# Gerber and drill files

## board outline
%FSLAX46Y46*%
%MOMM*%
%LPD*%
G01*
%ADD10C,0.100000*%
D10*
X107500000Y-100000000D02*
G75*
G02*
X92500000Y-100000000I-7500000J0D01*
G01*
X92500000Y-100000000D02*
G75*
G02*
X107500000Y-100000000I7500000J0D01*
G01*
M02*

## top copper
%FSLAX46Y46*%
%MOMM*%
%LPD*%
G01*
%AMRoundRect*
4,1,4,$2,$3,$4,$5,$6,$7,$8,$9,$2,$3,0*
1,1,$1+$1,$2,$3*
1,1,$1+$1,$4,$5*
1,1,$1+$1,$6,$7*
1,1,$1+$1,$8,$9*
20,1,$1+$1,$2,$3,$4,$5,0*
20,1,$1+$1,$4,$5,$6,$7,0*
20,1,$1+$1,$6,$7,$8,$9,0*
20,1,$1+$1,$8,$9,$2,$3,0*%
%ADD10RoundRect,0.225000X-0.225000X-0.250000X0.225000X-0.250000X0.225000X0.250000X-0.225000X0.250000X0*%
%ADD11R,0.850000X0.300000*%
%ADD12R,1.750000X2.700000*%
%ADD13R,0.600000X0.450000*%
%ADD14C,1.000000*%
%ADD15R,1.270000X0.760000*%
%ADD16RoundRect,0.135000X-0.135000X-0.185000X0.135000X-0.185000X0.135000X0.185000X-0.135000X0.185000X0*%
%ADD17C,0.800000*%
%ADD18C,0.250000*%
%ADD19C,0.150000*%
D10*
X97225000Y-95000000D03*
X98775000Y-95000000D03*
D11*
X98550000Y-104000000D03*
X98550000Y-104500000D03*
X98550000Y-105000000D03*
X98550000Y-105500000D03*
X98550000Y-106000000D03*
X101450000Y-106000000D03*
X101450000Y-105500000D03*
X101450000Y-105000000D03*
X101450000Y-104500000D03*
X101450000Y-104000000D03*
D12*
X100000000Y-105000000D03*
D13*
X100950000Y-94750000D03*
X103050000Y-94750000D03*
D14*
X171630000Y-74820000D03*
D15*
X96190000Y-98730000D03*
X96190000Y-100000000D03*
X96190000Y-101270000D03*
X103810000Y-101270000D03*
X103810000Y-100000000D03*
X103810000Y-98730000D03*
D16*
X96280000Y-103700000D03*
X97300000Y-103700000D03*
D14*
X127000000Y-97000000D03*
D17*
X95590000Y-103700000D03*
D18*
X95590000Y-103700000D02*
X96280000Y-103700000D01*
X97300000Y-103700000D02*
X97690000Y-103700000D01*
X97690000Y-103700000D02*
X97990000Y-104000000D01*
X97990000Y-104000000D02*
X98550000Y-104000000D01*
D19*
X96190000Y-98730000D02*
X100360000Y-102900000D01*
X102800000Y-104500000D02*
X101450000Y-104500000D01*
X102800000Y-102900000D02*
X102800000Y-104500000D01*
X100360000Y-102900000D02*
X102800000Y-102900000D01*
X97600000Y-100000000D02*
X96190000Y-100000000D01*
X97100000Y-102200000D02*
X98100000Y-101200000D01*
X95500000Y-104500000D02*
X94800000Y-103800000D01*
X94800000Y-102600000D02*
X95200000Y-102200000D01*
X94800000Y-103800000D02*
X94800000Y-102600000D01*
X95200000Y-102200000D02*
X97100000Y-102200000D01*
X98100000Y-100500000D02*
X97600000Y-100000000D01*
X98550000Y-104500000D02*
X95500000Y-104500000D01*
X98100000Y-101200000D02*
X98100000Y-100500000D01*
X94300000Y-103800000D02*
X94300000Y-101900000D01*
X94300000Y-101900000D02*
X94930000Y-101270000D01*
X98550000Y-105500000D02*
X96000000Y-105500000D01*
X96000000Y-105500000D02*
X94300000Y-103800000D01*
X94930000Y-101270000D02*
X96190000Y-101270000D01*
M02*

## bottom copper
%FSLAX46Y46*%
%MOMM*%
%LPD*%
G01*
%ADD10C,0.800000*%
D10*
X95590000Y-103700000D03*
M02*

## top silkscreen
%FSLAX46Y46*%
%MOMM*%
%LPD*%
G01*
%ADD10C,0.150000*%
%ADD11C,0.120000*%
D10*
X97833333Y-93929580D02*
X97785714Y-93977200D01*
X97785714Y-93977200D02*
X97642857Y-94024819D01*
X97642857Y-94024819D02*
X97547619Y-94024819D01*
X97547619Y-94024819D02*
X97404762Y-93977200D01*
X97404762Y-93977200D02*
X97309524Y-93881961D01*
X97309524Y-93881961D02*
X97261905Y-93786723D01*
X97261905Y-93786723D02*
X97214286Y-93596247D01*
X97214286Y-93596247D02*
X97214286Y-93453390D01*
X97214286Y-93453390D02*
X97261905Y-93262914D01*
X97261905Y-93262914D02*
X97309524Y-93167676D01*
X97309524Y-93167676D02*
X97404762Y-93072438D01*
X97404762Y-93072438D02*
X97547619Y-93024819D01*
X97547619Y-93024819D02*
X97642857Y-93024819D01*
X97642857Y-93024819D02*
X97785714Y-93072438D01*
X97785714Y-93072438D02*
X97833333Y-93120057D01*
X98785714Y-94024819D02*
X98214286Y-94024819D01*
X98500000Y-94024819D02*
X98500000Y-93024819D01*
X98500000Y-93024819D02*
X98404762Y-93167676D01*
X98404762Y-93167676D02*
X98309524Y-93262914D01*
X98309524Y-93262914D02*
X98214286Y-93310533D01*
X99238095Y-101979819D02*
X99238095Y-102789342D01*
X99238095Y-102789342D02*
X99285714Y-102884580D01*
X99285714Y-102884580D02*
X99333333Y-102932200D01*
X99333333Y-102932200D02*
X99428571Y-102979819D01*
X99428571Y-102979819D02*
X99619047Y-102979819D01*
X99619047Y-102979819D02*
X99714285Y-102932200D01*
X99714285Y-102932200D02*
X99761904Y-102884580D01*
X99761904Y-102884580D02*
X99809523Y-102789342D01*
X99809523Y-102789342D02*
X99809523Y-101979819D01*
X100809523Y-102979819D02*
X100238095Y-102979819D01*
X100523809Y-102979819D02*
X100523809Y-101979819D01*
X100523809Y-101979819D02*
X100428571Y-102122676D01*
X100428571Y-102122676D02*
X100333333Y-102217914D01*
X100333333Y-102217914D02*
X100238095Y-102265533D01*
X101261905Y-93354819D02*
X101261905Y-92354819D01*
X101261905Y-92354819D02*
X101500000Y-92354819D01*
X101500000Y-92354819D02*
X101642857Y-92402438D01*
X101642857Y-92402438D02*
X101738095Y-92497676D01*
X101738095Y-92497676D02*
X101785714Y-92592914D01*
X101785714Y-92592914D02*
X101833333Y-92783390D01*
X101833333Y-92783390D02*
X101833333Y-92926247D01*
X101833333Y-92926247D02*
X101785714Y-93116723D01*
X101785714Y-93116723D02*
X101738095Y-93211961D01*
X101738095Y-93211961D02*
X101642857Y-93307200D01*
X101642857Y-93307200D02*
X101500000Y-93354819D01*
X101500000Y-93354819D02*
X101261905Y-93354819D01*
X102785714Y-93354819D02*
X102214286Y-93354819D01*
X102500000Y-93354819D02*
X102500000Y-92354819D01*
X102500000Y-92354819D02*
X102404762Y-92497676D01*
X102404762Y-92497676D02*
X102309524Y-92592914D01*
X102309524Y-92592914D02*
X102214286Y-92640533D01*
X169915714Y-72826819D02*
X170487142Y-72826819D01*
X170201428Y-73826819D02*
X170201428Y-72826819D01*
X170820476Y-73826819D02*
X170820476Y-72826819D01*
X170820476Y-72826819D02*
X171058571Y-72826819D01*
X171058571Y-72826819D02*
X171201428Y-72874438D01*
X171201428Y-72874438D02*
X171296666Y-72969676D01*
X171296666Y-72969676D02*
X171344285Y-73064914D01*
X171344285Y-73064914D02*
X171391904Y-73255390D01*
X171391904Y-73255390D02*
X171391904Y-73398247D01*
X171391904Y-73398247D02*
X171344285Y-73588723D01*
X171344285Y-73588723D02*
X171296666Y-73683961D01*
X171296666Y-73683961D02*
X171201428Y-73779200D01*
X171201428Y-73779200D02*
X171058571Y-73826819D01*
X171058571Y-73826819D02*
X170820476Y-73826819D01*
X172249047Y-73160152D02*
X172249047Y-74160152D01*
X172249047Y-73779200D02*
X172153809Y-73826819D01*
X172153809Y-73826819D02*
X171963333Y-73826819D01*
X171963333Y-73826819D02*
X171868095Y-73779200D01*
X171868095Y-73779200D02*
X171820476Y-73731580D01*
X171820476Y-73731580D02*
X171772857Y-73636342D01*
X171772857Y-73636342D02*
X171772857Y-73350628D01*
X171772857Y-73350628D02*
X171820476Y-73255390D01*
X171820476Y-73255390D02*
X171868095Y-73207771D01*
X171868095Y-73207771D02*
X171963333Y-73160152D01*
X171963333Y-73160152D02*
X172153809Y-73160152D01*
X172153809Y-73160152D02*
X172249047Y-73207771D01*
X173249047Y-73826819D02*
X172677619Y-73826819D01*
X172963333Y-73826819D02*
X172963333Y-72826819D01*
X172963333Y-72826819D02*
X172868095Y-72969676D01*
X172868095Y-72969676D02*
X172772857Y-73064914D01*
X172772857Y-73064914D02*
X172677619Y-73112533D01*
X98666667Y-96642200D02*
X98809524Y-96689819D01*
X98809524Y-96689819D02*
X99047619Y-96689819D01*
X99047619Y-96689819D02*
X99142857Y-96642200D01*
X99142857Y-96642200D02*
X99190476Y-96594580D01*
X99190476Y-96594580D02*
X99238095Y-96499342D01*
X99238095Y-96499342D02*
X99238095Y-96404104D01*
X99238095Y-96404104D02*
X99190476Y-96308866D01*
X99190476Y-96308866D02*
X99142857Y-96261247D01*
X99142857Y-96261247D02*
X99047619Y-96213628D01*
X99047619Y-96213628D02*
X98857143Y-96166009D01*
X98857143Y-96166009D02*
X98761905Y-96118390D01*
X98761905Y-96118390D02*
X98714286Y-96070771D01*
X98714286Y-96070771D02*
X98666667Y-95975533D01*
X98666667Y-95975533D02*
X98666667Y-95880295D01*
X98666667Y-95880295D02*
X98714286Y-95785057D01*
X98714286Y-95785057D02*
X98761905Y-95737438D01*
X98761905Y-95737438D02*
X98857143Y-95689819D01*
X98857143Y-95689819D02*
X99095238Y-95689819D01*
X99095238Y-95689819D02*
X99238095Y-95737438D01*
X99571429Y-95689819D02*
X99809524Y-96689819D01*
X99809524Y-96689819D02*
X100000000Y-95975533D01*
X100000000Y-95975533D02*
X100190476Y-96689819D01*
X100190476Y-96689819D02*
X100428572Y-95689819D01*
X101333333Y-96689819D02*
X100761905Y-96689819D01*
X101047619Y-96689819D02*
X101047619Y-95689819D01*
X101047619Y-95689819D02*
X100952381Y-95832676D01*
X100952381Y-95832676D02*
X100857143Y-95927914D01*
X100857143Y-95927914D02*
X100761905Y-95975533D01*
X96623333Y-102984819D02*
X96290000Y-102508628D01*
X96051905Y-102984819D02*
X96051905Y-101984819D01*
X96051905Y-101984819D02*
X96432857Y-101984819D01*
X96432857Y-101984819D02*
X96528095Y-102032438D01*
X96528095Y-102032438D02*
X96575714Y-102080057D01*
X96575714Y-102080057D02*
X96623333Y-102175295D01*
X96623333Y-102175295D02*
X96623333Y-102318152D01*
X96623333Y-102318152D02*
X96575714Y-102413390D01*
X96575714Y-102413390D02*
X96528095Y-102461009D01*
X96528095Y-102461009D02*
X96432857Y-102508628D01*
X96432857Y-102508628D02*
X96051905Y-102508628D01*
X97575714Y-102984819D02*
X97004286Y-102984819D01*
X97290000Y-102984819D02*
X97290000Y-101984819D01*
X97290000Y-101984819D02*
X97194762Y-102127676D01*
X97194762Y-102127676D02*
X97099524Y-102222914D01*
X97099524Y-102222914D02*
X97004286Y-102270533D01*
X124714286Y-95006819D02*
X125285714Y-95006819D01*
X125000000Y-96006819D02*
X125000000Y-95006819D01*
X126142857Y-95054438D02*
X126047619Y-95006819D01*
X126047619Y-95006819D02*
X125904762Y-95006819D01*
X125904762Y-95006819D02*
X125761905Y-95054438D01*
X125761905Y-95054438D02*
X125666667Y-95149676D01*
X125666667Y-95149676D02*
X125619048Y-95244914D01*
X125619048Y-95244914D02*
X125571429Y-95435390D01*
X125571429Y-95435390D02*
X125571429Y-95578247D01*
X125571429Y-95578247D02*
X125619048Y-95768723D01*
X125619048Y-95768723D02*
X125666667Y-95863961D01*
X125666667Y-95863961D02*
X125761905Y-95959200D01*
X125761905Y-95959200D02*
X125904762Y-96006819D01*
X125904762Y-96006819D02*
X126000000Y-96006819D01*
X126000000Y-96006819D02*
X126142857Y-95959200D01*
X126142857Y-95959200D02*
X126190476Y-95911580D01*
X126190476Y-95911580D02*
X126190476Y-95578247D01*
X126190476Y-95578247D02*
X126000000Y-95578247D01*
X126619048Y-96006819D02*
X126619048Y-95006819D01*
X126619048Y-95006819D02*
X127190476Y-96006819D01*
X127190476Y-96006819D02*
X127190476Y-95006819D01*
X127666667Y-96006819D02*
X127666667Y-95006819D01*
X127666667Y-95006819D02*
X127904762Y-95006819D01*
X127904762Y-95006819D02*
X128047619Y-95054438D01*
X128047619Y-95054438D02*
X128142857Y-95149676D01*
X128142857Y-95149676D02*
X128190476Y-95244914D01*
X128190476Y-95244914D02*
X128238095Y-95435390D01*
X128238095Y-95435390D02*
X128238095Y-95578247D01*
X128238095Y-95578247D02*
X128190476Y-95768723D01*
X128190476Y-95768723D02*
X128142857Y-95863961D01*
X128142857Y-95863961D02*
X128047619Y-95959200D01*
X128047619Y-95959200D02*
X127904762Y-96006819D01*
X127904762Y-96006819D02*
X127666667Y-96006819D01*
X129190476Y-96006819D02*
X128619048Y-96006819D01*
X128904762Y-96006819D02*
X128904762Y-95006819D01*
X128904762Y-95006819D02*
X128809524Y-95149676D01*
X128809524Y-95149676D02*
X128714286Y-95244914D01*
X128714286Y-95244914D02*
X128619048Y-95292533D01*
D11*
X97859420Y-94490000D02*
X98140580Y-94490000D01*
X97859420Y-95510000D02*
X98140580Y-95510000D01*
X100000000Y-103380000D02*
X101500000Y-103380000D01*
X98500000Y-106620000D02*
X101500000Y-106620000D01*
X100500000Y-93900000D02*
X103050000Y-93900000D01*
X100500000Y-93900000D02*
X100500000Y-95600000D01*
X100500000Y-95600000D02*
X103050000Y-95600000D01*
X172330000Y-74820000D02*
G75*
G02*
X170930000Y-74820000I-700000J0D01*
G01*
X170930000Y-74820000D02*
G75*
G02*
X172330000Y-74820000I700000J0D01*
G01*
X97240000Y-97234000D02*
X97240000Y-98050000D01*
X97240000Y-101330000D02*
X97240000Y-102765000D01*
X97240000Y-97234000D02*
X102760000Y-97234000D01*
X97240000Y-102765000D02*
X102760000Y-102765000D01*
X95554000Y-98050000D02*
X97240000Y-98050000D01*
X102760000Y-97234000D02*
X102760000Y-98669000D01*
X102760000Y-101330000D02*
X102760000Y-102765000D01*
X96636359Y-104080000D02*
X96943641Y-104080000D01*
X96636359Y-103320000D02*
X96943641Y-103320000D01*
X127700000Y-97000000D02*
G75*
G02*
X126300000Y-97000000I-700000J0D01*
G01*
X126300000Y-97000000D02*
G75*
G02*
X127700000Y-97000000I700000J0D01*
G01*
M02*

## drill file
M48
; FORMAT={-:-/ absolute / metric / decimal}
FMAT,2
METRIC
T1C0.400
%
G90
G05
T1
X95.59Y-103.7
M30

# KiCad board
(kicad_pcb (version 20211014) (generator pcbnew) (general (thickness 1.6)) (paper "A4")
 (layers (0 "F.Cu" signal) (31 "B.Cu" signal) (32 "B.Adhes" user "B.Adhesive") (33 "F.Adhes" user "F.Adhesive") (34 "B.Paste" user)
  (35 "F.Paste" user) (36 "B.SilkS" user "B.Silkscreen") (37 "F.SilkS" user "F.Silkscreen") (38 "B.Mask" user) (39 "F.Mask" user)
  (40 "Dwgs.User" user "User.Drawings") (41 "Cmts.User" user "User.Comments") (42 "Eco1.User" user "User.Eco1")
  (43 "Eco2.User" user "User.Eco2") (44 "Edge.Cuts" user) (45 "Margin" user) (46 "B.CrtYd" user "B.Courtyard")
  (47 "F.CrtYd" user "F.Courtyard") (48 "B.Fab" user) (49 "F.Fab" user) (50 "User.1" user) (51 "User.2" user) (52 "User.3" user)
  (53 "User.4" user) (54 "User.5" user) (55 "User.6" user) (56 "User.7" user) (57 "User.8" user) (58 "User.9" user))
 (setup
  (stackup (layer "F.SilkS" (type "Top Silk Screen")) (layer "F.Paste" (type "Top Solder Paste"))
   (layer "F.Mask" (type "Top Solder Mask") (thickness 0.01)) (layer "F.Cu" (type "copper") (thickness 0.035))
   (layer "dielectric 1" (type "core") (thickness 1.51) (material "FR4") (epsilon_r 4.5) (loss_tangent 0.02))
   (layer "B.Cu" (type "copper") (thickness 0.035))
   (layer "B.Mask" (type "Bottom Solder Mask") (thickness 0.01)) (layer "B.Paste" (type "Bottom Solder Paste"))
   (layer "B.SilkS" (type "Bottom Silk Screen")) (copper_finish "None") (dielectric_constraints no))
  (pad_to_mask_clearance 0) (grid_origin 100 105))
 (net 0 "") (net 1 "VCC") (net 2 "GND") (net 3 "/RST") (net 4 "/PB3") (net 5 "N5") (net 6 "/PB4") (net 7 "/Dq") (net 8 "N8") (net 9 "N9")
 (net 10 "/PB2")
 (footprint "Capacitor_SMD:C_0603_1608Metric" (layer "F.Cu") (at 98 95)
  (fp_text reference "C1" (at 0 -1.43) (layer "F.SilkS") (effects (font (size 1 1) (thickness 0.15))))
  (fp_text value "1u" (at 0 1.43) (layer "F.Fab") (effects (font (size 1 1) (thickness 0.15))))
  (fp_line (start -0.14058 -0.51) (end 0.14058 -0.51) (layer "F.SilkS") (width 0.12))
  (fp_line (start -0.14058 0.51) (end 0.14058 0.51) (layer "F.SilkS") (width 0.12))
  (pad "1" smd roundrect locked (at -0.775 0) (size 0.9 0.95) (layers "F.Cu" "F.Paste" "F.Mask") (roundrect_rratio 0.25) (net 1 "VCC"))
  (pad "2" smd roundrect locked (at 0.775 0) (size 0.9 0.95) (layers "F.Cu" "F.Paste" "F.Mask") (roundrect_rratio 0.25) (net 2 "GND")))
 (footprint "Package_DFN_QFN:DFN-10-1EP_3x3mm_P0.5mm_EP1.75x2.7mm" (layer "F.Cu") (at 100 105)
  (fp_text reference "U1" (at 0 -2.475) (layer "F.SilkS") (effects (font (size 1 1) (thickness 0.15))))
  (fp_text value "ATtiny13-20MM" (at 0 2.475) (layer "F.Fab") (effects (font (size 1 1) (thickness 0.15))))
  (fp_line (start 0 -1.62) (end 1.5 -1.62) (layer "F.SilkS") (width 0.12))
  (fp_line (start -1.5 1.62) (end 1.5 1.62) (layer "F.SilkS") (width 0.12))
  (pad "" smd rect locked (at 0.3875 0.62) (size 0.6 1.05) (layers "F.Paste"))
  (pad "" smd rect locked (at -0.3875 0.62) (size 0.6 1.05) (layers "F.Paste"))
  (pad "" smd rect locked (at 0.3875 -0.62) (size 0.6 1.05) (layers "F.Paste"))
  (pad "" smd rect locked (at -0.3875 -0.62) (size 0.6 1.05) (layers "F.Paste"))
  (pad "1" smd rect locked (at -1.45 -1) (size 0.85 0.3) (layers "F.Cu" "F.Paste" "F.Mask") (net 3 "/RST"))
  (pad "2" smd rect locked (at -1.45 -0.5) (size 0.85 0.3) (layers "F.Cu" "F.Paste" "F.Mask") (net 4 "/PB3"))
  (pad "3" smd rect locked (at -1.45 0) (size 0.85 0.3) (layers "F.Cu" "F.Paste" "F.Mask") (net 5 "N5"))
  (pad "4" smd rect locked (at -1.45 0.5) (size 0.85 0.3) (layers "F.Cu" "F.Paste" "F.Mask") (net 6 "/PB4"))
  (pad "5" smd rect locked (at -1.45 1) (size 0.85 0.3) (layers "F.Cu" "F.Paste" "F.Mask") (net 2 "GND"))
  (pad "6" smd rect locked (at 1.45 1) (size 0.85 0.3) (layers "F.Cu" "F.Paste" "F.Mask") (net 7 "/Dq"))
  (pad "7" smd rect locked (at 1.45 0.5) (size 0.85 0.3) (layers "F.Cu" "F.Paste" "F.Mask") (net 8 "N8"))
  (pad "8" smd rect locked (at 1.45 0) (size 0.85 0.3) (layers "F.Cu" "F.Paste" "F.Mask") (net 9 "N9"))
  (pad "9" smd rect locked (at 1.45 -0.5) (size 0.85 0.3) (layers "F.Cu" "F.Paste" "F.Mask") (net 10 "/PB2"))
  (pad "10" smd rect locked (at 1.45 -1) (size 0.85 0.3) (layers "F.Cu" "F.Paste" "F.Mask") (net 1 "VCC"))
  (pad "11" smd rect locked (at 0 0) (size 1.75 2.7) (layers "F.Cu" "F.Mask") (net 2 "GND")))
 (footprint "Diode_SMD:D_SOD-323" (layer "F.Cu") (at 102 94.75)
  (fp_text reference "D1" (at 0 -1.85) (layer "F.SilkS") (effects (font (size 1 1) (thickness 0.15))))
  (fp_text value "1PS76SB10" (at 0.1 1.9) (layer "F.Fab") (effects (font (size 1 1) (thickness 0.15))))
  (fp_line (start -1.5 -0.85) (end 1.05 -0.85) (layer "F.SilkS") (width 0.12))
  (fp_line (start -1.5 -0.85) (end -1.5 0.85) (layer "F.SilkS") (width 0.12))
  (fp_line (start -1.5 0.85) (end 1.05 0.85) (layer "F.SilkS") (width 0.12))
  (pad "1" smd rect locked (at -1.05 0) (size 0.6 0.45) (layers "F.Cu" "F.Paste" "F.Mask") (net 1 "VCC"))
  (pad "2" smd rect locked (at 1.05 0) (size 0.6 0.45) (layers "F.Cu" "F.Paste" "F.Mask") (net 7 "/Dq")))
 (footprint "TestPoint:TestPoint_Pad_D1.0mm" (layer "F.Cu") (at 171.63 74.82)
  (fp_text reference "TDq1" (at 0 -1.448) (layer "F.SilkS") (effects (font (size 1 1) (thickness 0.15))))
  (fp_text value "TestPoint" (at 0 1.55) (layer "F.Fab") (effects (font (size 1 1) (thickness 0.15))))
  (fp_circle (center 0 0) (end 0 0.7) (layer "F.SilkS") (width 0.12) (fill none))
  (pad "1" smd circle locked (at 0 0) (size 1 1) (layers "F.Cu" "F.Mask") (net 7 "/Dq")))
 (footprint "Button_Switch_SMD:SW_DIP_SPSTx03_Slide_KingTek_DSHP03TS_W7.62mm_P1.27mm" (layer "F.Cu") (at 100 100)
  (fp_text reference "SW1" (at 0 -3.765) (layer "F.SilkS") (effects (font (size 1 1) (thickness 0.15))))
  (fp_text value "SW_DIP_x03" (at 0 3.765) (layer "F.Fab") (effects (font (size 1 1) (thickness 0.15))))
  (fp_line (start -2.76 -2.766) (end -2.76 -1.95) (layer "F.SilkS") (width 0.12))
  (fp_line (start -2.76 1.33) (end -2.76 2.765) (layer "F.SilkS") (width 0.12))
  (fp_line (start -2.76 -2.766) (end 2.76 -2.766) (layer "F.SilkS") (width 0.12))
  (fp_line (start -2.76 2.765) (end 2.76 2.765) (layer "F.SilkS") (width 0.12))
  (fp_line (start -4.446 -1.95) (end -2.76 -1.95) (layer "F.SilkS") (width 0.12))
  (fp_line (start 2.76 -2.766) (end 2.76 -1.331) (layer "F.SilkS") (width 0.12))
  (fp_line (start 2.76 1.33) (end 2.76 2.765) (layer "F.SilkS") (width 0.12))
  (pad "1" smd rect locked (at -3.81 -1.27) (size 1.27 0.76) (layers "F.Cu" "F.Paste" "F.Mask") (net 10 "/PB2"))
  (pad "2" smd rect locked (at -3.81 0) (size 1.27 0.76) (layers "F.Cu" "F.Paste" "F.Mask") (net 4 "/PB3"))
  (pad "3" smd rect locked (at -3.81 1.27) (size 1.27 0.76) (layers "F.Cu" "F.Paste" "F.Mask") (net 6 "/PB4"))
  (pad "4" smd rect locked (at 3.81 1.27) (size 1.27 0.76) (layers "F.Cu" "F.Paste" "F.Mask") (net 2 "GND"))
  (pad "5" smd rect locked (at 3.81 0) (size 1.27 0.76) (layers "F.Cu" "F.Paste" "F.Mask") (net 2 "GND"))
  (pad "6" smd rect locked (at 3.81 -1.27) (size 1.27 0.76) (layers "F.Cu" "F.Paste" "F.Mask") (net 2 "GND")))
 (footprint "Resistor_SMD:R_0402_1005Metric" (layer "F.Cu") (at 96.79 103.7)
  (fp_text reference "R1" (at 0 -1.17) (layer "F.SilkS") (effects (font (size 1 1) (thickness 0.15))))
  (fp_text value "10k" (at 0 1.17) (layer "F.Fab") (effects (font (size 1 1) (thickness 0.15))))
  (fp_line (start -0.153641 0.38) (end 0.153641 0.38) (layer "F.SilkS") (width 0.12))
  (fp_line (start -0.153641 -0.38) (end 0.153641 -0.38) (layer "F.SilkS") (width 0.12))
  (pad "1" smd roundrect locked (at -0.51 0) (size 0.54 0.64) (layers "F.Cu" "F.Paste" "F.Mask") (roundrect_rratio 0.25) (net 1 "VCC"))
  (pad "2" smd roundrect locked (at 0.51 0) (size 0.54 0.64) (layers "F.Cu" "F.Paste" "F.Mask") (roundrect_rratio 0.25) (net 3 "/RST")))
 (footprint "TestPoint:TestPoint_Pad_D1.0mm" (layer "F.Cu") (at 127 97)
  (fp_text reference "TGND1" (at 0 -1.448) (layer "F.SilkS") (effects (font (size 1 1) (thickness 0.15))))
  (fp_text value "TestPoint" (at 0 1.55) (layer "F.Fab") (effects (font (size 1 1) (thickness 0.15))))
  (fp_circle (center 0 0) (end 0 0.7) (layer "F.SilkS") (width 0.12) (fill none))
  (pad "1" smd circle locked (at 0 0) (size 1 1) (layers "F.Cu" "F.Mask") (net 2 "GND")))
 (gr_circle (center 100 100) (end 107.5 100) (layer "Edge.Cuts") (width 0.1) (fill none))
 (segment (start 95.59 103.7) (end 96.28 103.7) (width 0.25) (layer "F.Cu") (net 1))
 (via (at 95.59 103.7) (size 0.8) (drill 0.4) (layers "F.Cu" "B.Cu") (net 1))
 (segment (start 97.3 103.7) (end 97.69 103.7) (width 0.25) (layer "F.Cu") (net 3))
 (segment (start 97.69 103.7) (end 97.99 104) (width 0.25) (layer "F.Cu") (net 3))
 (segment (start 97.99 104) (end 98.55 104) (width 0.25) (layer "F.Cu") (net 3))
 (segment (start 96.19 98.73) (end 100.36 102.9) (width 0.15) (layer "F.Cu") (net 10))
 (segment (start 102.8 104.5) (end 101.45 104.5) (width 0.15) (layer "F.Cu") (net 10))
 (segment (start 102.8 102.9) (end 102.8 104.5) (width 0.15) (layer "F.Cu") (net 10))
 (segment (start 100.36 102.9) (end 102.8 102.9) (width 0.15) (layer "F.Cu") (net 10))
 (segment (start 97.6 100) (end 96.19 100) (width 0.15) (layer "F.Cu") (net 4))
 (segment (start 97.1 102.2) (end 98.1 101.2) (width 0.15) (layer "F.Cu") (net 4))
 (segment (start 95.5 104.5) (end 94.8 103.8) (width 0.15) (layer "F.Cu") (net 4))
 (segment (start 94.8 102.6) (end 95.2 102.2) (width 0.15) (layer "F.Cu") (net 4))
 (segment (start 94.8 103.8) (end 94.8 102.6) (width 0.15) (layer "F.Cu") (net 4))
 (segment (start 95.2 102.2) (end 97.1 102.2) (width 0.15) (layer "F.Cu") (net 4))
 (segment (start 98.1 100.5) (end 97.6 100) (width 0.15) (layer "F.Cu") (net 4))
 (segment (start 98.55 104.5) (end 95.5 104.5) (width 0.15) (layer "F.Cu") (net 4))
 (segment (start 98.1 101.2) (end 98.1 100.5) (width 0.15) (layer "F.Cu") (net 4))
 (segment (start 94.3 103.8) (end 94.3 101.9) (width 0.15) (layer "F.Cu") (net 6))
 (segment (start 94.3 101.9) (end 94.93 101.27) (width 0.15) (layer "F.Cu") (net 6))
 (segment (start 98.55 105.5) (end 96 105.5) (width 0.15) (layer "F.Cu") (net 6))
 (segment (start 96 105.5) (end 94.3 103.8) (width 0.15) (layer "F.Cu") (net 6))
 (segment (start 94.93 101.27) (end 96.19 101.27) (width 0.15) (layer "F.Cu") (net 6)))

